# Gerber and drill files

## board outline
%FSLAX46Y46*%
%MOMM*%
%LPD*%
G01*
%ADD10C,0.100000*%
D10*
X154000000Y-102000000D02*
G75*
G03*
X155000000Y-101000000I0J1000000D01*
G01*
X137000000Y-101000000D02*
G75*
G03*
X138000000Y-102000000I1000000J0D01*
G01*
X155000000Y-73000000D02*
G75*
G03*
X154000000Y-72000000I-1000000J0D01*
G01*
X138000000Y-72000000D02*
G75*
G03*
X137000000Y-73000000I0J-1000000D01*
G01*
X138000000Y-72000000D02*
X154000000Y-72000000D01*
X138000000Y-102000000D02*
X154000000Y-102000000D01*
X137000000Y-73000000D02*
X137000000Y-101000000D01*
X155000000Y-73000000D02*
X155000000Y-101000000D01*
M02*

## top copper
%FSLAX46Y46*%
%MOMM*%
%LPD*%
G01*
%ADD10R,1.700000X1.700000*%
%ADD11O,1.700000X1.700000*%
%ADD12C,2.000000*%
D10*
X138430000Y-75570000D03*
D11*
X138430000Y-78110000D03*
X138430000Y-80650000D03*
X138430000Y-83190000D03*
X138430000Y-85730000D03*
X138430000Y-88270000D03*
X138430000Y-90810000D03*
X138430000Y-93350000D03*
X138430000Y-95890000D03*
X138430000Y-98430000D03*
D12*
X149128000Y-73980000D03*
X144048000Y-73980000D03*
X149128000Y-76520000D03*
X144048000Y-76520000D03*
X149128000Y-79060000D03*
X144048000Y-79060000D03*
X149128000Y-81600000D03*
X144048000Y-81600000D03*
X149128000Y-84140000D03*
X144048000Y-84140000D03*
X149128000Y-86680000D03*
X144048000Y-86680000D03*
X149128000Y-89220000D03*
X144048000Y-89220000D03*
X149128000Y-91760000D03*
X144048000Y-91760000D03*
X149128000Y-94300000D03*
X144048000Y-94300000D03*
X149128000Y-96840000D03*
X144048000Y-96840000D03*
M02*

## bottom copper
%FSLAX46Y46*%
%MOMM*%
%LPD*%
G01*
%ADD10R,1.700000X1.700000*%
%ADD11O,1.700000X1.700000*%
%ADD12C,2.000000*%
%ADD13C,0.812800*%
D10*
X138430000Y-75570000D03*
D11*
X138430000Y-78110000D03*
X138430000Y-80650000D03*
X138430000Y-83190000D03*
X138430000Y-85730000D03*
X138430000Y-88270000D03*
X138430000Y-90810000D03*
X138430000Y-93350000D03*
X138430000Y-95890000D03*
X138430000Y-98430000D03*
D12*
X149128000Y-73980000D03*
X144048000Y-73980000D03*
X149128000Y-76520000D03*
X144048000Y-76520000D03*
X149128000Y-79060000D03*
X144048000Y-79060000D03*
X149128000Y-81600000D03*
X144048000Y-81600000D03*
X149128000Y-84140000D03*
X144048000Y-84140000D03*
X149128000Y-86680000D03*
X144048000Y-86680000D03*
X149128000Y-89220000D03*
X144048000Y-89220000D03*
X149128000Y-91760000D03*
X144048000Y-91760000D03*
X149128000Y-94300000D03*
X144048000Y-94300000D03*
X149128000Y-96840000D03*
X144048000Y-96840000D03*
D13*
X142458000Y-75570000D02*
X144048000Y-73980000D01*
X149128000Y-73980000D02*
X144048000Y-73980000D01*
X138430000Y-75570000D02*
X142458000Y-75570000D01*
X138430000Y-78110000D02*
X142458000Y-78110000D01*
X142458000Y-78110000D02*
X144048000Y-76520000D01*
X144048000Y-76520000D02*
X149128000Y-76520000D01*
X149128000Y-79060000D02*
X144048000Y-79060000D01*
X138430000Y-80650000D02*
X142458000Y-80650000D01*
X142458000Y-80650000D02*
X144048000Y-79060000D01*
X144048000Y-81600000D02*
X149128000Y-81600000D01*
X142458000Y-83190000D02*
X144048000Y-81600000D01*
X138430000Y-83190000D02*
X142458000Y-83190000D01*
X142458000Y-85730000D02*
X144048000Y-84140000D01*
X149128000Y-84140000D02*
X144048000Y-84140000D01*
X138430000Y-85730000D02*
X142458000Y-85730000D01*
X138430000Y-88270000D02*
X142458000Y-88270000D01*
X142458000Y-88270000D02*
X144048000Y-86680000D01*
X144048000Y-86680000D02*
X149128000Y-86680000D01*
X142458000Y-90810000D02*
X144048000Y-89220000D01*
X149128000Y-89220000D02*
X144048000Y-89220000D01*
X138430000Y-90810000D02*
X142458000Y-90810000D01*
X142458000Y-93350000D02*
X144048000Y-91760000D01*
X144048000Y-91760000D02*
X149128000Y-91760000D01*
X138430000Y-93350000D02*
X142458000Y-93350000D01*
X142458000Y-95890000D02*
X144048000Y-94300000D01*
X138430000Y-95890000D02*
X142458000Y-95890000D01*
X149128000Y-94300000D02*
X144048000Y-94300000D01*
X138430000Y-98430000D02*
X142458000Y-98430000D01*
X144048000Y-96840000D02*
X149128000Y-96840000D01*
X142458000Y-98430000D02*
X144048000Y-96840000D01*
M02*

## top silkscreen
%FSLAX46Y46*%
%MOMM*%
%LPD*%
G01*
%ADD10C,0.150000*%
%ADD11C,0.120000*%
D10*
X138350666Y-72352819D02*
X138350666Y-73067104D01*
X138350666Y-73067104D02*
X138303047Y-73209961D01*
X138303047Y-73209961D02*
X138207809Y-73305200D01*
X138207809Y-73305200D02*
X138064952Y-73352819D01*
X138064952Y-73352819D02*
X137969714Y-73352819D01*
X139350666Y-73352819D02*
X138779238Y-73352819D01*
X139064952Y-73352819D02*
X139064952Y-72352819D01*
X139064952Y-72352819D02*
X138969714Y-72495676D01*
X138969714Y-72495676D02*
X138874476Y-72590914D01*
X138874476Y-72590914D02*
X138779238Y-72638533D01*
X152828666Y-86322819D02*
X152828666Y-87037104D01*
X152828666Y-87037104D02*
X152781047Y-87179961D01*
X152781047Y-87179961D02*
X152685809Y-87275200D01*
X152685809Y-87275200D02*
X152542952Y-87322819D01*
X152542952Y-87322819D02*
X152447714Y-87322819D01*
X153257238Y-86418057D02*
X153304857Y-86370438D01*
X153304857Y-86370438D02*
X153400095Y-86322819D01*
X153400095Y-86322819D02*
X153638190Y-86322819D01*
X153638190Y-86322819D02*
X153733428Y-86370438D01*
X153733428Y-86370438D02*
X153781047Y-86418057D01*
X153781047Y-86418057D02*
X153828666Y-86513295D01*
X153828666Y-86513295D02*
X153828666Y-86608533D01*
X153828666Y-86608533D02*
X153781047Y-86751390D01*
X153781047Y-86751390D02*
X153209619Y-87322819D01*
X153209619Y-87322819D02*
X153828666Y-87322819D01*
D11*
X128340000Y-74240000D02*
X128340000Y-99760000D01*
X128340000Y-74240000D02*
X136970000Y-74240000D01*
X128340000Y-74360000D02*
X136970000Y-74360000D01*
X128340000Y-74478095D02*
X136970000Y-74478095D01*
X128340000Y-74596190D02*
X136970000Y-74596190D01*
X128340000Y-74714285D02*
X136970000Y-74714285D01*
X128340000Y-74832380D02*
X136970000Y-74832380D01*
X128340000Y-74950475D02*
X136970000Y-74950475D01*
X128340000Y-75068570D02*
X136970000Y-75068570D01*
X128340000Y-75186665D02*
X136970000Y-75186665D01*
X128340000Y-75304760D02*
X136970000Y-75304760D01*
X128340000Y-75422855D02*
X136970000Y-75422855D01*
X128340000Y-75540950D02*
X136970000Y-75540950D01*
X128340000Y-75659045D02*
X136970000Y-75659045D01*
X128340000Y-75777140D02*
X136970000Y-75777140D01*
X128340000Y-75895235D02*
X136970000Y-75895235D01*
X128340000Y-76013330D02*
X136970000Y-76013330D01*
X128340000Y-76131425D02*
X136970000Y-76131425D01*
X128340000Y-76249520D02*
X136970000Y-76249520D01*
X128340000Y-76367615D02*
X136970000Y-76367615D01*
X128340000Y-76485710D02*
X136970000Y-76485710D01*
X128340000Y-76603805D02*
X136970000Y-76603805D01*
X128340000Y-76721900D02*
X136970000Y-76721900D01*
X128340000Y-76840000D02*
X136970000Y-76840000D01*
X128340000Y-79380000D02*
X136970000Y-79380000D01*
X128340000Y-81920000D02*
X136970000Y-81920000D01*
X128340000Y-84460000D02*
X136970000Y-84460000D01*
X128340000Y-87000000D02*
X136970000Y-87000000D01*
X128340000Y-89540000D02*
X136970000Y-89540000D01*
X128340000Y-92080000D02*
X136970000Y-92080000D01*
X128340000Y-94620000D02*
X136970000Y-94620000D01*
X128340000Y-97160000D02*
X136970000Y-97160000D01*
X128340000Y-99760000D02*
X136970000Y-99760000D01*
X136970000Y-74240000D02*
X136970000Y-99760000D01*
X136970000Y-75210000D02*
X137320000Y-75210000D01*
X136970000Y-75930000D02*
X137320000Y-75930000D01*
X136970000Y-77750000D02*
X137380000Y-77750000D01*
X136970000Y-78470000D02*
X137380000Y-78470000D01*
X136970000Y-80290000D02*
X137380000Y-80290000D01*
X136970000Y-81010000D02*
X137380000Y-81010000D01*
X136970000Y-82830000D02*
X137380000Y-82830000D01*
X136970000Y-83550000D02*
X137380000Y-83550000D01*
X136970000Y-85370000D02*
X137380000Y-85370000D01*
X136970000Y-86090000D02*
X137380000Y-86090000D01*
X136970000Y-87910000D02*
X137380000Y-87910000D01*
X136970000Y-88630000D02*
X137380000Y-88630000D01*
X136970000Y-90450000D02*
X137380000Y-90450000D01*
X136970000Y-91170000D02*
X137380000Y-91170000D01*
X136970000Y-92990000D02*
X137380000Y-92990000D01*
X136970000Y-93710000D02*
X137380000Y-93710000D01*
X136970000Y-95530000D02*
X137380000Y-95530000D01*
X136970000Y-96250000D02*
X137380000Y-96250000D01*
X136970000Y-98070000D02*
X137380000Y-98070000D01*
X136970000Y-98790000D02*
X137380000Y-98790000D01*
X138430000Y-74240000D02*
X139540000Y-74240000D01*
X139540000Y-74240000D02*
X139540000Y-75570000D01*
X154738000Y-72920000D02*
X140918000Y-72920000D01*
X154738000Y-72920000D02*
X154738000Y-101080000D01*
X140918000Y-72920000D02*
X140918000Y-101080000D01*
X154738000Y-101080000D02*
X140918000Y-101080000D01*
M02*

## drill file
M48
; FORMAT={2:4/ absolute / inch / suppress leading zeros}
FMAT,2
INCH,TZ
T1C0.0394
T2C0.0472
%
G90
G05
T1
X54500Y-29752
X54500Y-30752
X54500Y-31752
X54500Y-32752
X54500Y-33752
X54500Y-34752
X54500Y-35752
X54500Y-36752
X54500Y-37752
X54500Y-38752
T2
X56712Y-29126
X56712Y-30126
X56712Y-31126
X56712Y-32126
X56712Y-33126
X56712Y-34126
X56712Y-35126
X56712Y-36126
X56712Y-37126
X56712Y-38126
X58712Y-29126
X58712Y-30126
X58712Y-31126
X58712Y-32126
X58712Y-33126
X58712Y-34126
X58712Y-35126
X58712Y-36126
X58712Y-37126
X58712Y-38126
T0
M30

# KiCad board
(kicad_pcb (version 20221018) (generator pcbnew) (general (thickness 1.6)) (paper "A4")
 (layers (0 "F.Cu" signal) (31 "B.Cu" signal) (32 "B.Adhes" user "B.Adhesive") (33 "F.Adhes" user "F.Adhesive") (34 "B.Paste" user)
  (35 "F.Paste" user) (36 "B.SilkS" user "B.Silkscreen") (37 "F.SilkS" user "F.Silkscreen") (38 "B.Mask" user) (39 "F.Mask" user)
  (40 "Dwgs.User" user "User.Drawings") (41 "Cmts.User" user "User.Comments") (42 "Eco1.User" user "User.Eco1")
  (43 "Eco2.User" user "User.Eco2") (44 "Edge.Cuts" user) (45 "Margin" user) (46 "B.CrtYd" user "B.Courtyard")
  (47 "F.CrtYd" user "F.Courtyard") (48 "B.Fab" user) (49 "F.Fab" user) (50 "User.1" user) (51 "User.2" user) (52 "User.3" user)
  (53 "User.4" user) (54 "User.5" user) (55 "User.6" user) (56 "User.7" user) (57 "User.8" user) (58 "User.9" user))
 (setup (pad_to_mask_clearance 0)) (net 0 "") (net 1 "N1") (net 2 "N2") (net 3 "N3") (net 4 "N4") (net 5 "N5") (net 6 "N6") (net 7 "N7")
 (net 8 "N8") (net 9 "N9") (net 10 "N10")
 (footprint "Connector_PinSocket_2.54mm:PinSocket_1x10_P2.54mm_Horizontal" (layer "F.Cu") (at 138.43 75.57)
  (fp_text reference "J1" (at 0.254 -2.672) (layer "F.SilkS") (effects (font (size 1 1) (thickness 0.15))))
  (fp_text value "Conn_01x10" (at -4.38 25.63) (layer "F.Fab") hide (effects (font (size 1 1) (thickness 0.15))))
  (fp_line (start -10.09 -1.33) (end -10.09 24.19) (stroke (width 0.12) (type solid)) (layer "F.SilkS"))
  (fp_line (start -10.09 -1.33) (end -1.46 -1.33) (stroke (width 0.12) (type solid)) (layer "F.SilkS"))
  (fp_line (start -10.09 -1.21) (end -1.46 -1.21) (stroke (width 0.12) (type solid)) (layer "F.SilkS"))
  (fp_line (start -10.09 -1.091905) (end -1.46 -1.091905) (stroke (width 0.12) (type solid)) (layer "F.SilkS"))
  (fp_line (start -10.09 -0.97381) (end -1.46 -0.97381) (stroke (width 0.12) (type solid)) (layer "F.SilkS"))
  (fp_line (start -10.09 -0.855715) (end -1.46 -0.855715) (stroke (width 0.12) (type solid)) (layer "F.SilkS"))
  (fp_line (start -10.09 -0.73762) (end -1.46 -0.73762) (stroke (width 0.12) (type solid)) (layer "F.SilkS"))
  (fp_line (start -10.09 -0.619525) (end -1.46 -0.619525) (stroke (width 0.12) (type solid)) (layer "F.SilkS"))
  (fp_line (start -10.09 -0.50143) (end -1.46 -0.50143) (stroke (width 0.12) (type solid)) (layer "F.SilkS"))
  (fp_line (start -10.09 -0.383335) (end -1.46 -0.383335) (stroke (width 0.12) (type solid)) (layer "F.SilkS"))
  (fp_line (start -10.09 -0.26524) (end -1.46 -0.26524) (stroke (width 0.12) (type solid)) (layer "F.SilkS"))
  (fp_line (start -10.09 -0.147145) (end -1.46 -0.147145) (stroke (width 0.12) (type solid)) (layer "F.SilkS"))
  (fp_line (start -10.09 -0.02905) (end -1.46 -0.02905) (stroke (width 0.12) (type solid)) (layer "F.SilkS"))
  (fp_line (start -10.09 0.089045) (end -1.46 0.089045) (stroke (width 0.12) (type solid)) (layer "F.SilkS"))
  (fp_line (start -10.09 0.20714) (end -1.46 0.20714) (stroke (width 0.12) (type solid)) (layer "F.SilkS"))
  (fp_line (start -10.09 0.325235) (end -1.46 0.325235) (stroke (width 0.12) (type solid)) (layer "F.SilkS"))
  (fp_line (start -10.09 0.44333) (end -1.46 0.44333) (stroke (width 0.12) (type solid)) (layer "F.SilkS"))
  (fp_line (start -10.09 0.561425) (end -1.46 0.561425) (stroke (width 0.12) (type solid)) (layer "F.SilkS"))
  (fp_line (start -10.09 0.67952) (end -1.46 0.67952) (stroke (width 0.12) (type solid)) (layer "F.SilkS"))
  (fp_line (start -10.09 0.797615) (end -1.46 0.797615) (stroke (width 0.12) (type solid)) (layer "F.SilkS"))
  (fp_line (start -10.09 0.91571) (end -1.46 0.91571) (stroke (width 0.12) (type solid)) (layer "F.SilkS"))
  (fp_line (start -10.09 1.033805) (end -1.46 1.033805) (stroke (width 0.12) (type solid)) (layer "F.SilkS"))
  (fp_line (start -10.09 1.1519) (end -1.46 1.1519) (stroke (width 0.12) (type solid)) (layer "F.SilkS"))
  (fp_line (start -10.09 1.27) (end -1.46 1.27) (stroke (width 0.12) (type solid)) (layer "F.SilkS"))
  (fp_line (start -10.09 3.81) (end -1.46 3.81) (stroke (width 0.12) (type solid)) (layer "F.SilkS"))
  (fp_line (start -10.09 6.35) (end -1.46 6.35) (stroke (width 0.12) (type solid)) (layer "F.SilkS"))
  (fp_line (start -10.09 8.89) (end -1.46 8.89) (stroke (width 0.12) (type solid)) (layer "F.SilkS"))
  (fp_line (start -10.09 11.43) (end -1.46 11.43) (stroke (width 0.12) (type solid)) (layer "F.SilkS"))
  (fp_line (start -10.09 13.97) (end -1.46 13.97) (stroke (width 0.12) (type solid)) (layer "F.SilkS"))
  (fp_line (start -10.09 16.51) (end -1.46 16.51) (stroke (width 0.12) (type solid)) (layer "F.SilkS"))
  (fp_line (start -10.09 19.05) (end -1.46 19.05) (stroke (width 0.12) (type solid)) (layer "F.SilkS"))
  (fp_line (start -10.09 21.59) (end -1.46 21.59) (stroke (width 0.12) (type solid)) (layer "F.SilkS"))
  (fp_line (start -10.09 24.19) (end -1.46 24.19) (stroke (width 0.12) (type solid)) (layer "F.SilkS"))
  (fp_line (start -1.46 -1.33) (end -1.46 24.19) (stroke (width 0.12) (type solid)) (layer "F.SilkS"))
  (fp_line (start -1.46 -0.36) (end -1.11 -0.36) (stroke (width 0.12) (type solid)) (layer "F.SilkS"))
  (fp_line (start -1.46 0.36) (end -1.11 0.36) (stroke (width 0.12) (type solid)) (layer "F.SilkS"))
  (fp_line (start -1.46 2.18) (end -1.05 2.18) (stroke (width 0.12) (type solid)) (layer "F.SilkS"))
  (fp_line (start -1.46 2.9) (end -1.05 2.9) (stroke (width 0.12) (type solid)) (layer "F.SilkS"))
  (fp_line (start -1.46 4.72) (end -1.05 4.72) (stroke (width 0.12) (type solid)) (layer "F.SilkS"))
  (fp_line (start -1.46 5.44) (end -1.05 5.44) (stroke (width 0.12) (type solid)) (layer "F.SilkS"))
  (fp_line (start -1.46 7.26) (end -1.05 7.26) (stroke (width 0.12) (type solid)) (layer "F.SilkS"))
  (fp_line (start -1.46 7.98) (end -1.05 7.98) (stroke (width 0.12) (type solid)) (layer "F.SilkS"))
  (fp_line (start -1.46 9.8) (end -1.05 9.8) (stroke (width 0.12) (type solid)) (layer "F.SilkS"))
  (fp_line (start -1.46 10.52) (end -1.05 10.52) (stroke (width 0.12) (type solid)) (layer "F.SilkS"))
  (fp_line (start -1.46 12.34) (end -1.05 12.34) (stroke (width 0.12) (type solid)) (layer "F.SilkS"))
  (fp_line (start -1.46 13.06) (end -1.05 13.06) (stroke (width 0.12) (type solid)) (layer "F.SilkS"))
  (fp_line (start -1.46 14.88) (end -1.05 14.88) (stroke (width 0.12) (type solid)) (layer "F.SilkS"))
  (fp_line (start -1.46 15.6) (end -1.05 15.6) (stroke (width 0.12) (type solid)) (layer "F.SilkS"))
  (fp_line (start -1.46 17.42) (end -1.05 17.42) (stroke (width 0.12) (type solid)) (layer "F.SilkS"))
  (fp_line (start -1.46 18.14) (end -1.05 18.14) (stroke (width 0.12) (type solid)) (layer "F.SilkS"))
  (fp_line (start -1.46 19.96) (end -1.05 19.96) (stroke (width 0.12) (type solid)) (layer "F.SilkS"))
  (fp_line (start -1.46 20.68) (end -1.05 20.68) (stroke (width 0.12) (type solid)) (layer "F.SilkS"))
  (fp_line (start -1.46 22.5) (end -1.05 22.5) (stroke (width 0.12) (type solid)) (layer "F.SilkS"))
  (fp_line (start -1.46 23.22) (end -1.05 23.22) (stroke (width 0.12) (type solid)) (layer "F.SilkS"))
  (fp_line (start 0 -1.33) (end 1.11 -1.33) (stroke (width 0.12) (type solid)) (layer "F.SilkS"))
  (fp_line (start 1.11 -1.33) (end 1.11 0) (stroke (width 0.12) (type solid)) (layer "F.SilkS"))
  (pad "1" thru_hole rect (at 0 0) (size 1.7 1.7) (drill 1) (layers "*.Cu" "*.Mask") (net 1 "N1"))
  (pad "2" thru_hole oval (at 0 2.54) (size 1.7 1.7) (drill 1) (layers "*.Cu" "*.Mask") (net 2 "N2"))
  (pad "3" thru_hole oval (at 0 5.08) (size 1.7 1.7) (drill 1) (layers "*.Cu" "*.Mask") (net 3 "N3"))
  (pad "4" thru_hole oval (at 0 7.62) (size 1.7 1.7) (drill 1) (layers "*.Cu" "*.Mask") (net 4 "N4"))
  (pad "5" thru_hole oval (at 0 10.16) (size 1.7 1.7) (drill 1) (layers "*.Cu" "*.Mask") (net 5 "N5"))
  (pad "6" thru_hole oval (at 0 12.7) (size 1.7 1.7) (drill 1) (layers "*.Cu" "*.Mask") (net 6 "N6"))
  (pad "7" thru_hole oval (at 0 15.24) (size 1.7 1.7) (drill 1) (layers "*.Cu" "*.Mask") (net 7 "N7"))
  (pad "8" thru_hole oval (at 0 17.78) (size 1.7 1.7) (drill 1) (layers "*.Cu" "*.Mask") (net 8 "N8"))
  (pad "9" thru_hole oval (at 0 20.32) (size 1.7 1.7) (drill 1) (layers "*.Cu" "*.Mask") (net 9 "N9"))
  (pad "10" thru_hole oval (at 0 22.86) (size 1.7 1.7) (drill 1) (layers "*.Cu" "*.Mask") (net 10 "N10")))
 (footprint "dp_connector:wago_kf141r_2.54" (layer "F.Cu") (at 147.828 87 -90)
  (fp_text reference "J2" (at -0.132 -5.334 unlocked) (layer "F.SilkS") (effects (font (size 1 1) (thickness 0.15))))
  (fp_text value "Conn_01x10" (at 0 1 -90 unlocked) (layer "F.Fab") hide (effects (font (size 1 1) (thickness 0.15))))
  (fp_line (start -14.08 -6.91) (end -14.08 6.91) (stroke (width 0.12) (type default)) (layer "F.SilkS"))
  (fp_line (start -14.08 -6.91) (end 14.08 -6.91) (stroke (width 0.12) (type default)) (layer "F.SilkS"))
  (fp_line (start -14.08 6.91) (end 14.08 6.91) (stroke (width 0.12) (type default)) (layer "F.SilkS"))
  (fp_line (start 14.08 -6.91) (end 14.08 6.91) (stroke (width 0.12) (type default)) (layer "F.SilkS"))
  (pad "1" thru_hole circle (at -13.02 -1.3 270) (size 2 2) (drill 1.2) (layers "*.Cu" "*.Mask") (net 1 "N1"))
  (pad "1" thru_hole circle (at -13.02 3.78 270) (size 2 2) (drill 1.2) (layers "*.Cu" "*.Mask") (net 1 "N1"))
  (pad "2" thru_hole circle (at -10.48 -1.3 270) (size 2 2) (drill 1.2) (layers "*.Cu" "*.Mask") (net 2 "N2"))
  (pad "2" thru_hole circle (at -10.48 3.78 270) (size 2 2) (drill 1.2) (layers "*.Cu" "*.Mask") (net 2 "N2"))
  (pad "3" thru_hole circle (at -7.94 -1.3 270) (size 2 2) (drill 1.2) (layers "*.Cu" "*.Mask") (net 3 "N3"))
  (pad "3" thru_hole circle (at -7.94 3.78 270) (size 2 2) (drill 1.2) (layers "*.Cu" "*.Mask") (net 3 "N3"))
  (pad "4" thru_hole circle (at -5.4 -1.3 270) (size 2 2) (drill 1.2) (layers "*.Cu" "*.Mask") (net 4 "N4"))
  (pad "4" thru_hole circle (at -5.4 3.78 270) (size 2 2) (drill 1.2) (layers "*.Cu" "*.Mask") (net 4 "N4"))
  (pad "5" thru_hole circle (at -2.86 -1.3 270) (size 2 2) (drill 1.2) (layers "*.Cu" "*.Mask") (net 5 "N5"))
  (pad "5" thru_hole circle (at -2.86 3.78 270) (size 2 2) (drill 1.2) (layers "*.Cu" "*.Mask") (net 5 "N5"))
  (pad "6" thru_hole circle (at -0.32 -1.3 270) (size 2 2) (drill 1.2) (layers "*.Cu" "*.Mask") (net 6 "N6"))
  (pad "6" thru_hole circle (at -0.32 3.78 270) (size 2 2) (drill 1.2) (layers "*.Cu" "*.Mask") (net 6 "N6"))
  (pad "7" thru_hole circle (at 2.22 -1.3 270) (size 2 2) (drill 1.2) (layers "*.Cu" "*.Mask") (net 7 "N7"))
  (pad "7" thru_hole circle (at 2.22 3.78 270) (size 2 2) (drill 1.2) (layers "*.Cu" "*.Mask") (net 7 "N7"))
  (pad "8" thru_hole circle (at 4.76 -1.3 270) (size 2 2) (drill 1.2) (layers "*.Cu" "*.Mask") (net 8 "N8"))
  (pad "8" thru_hole circle (at 4.76 3.78 270) (size 2 2) (drill 1.2) (layers "*.Cu" "*.Mask") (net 8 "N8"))
  (pad "9" thru_hole circle (at 7.3 -1.3 270) (size 2 2) (drill 1.2) (layers "*.Cu" "*.Mask") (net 9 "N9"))
  (pad "9" thru_hole circle (at 7.3 3.78 270) (size 2 2) (drill 1.2) (layers "*.Cu" "*.Mask") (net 9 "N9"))
  (pad "10" thru_hole circle (at 9.84 -1.3 270) (size 2 2) (drill 1.2) (layers "*.Cu" "*.Mask") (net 10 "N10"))
  (pad "10" thru_hole circle (at 9.84 3.78 270) (size 2 2) (drill 1.2) (layers "*.Cu" "*.Mask") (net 10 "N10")))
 (gr_line (start 138 72) (end 154 72) (stroke (width 0.1) (type default)) (layer "Edge.Cuts"))
 (gr_line (start 138 102) (end 154 102) (stroke (width 0.1) (type default)) (layer "Edge.Cuts"))
 (gr_line (start 137 73) (end 137 101) (stroke (width 0.1) (type default)) (layer "Edge.Cuts"))
 (gr_arc (start 155 101) (mid 154.707107 101.707107) (end 154 102) (stroke (width 0.1) (type default)) (layer "Edge.Cuts"))
 (gr_arc (start 154 72) (mid 154.707107 72.292893) (end 155 73) (stroke (width 0.1) (type default)) (layer "Edge.Cuts"))
 (gr_line (start 155 73) (end 155 101) (stroke (width 0.1) (type default)) (layer "Edge.Cuts"))
 (gr_arc (start 138 102) (mid 137.292893 101.707107) (end 137 101) (stroke (width 0.1) (type default)) (layer "Edge.Cuts"))
 (gr_arc (start 137 73) (mid 137.292893 72.292893) (end 138 72) (stroke (width 0.1) (type default)) (layer "Edge.Cuts"))
 (segment (start 142.458 75.57) (end 144.048 73.98) (width 0.8128) (layer "B.Cu") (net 1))
 (segment (start 149.128 73.98) (end 144.048 73.98) (width 0.8128) (layer "B.Cu") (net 1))
 (segment (start 138.43 75.57) (end 142.458 75.57) (width 0.8128) (layer "B.Cu") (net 1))
 (segment (start 138.43 78.11) (end 142.458 78.11) (width 0.8128) (layer "B.Cu") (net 2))
 (segment (start 142.458 78.11) (end 144.048 76.52) (width 0.8128) (layer "B.Cu") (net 2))
 (segment (start 144.048 76.52) (end 149.128 76.52) (width 0.8128) (layer "B.Cu") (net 2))
 (segment (start 149.128 79.06) (end 144.048 79.06) (width 0.8128) (layer "B.Cu") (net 3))
 (segment (start 138.43 80.65) (end 142.458 80.65) (width 0.8128) (layer "B.Cu") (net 3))
 (segment (start 142.458 80.65) (end 144.048 79.06) (width 0.8128) (layer "B.Cu") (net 3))
 (segment (start 144.048 81.6) (end 149.128 81.6) (width 0.8128) (layer "B.Cu") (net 4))
 (segment (start 142.458 83.19) (end 144.048 81.6) (width 0.8128) (layer "B.Cu") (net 4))
 (segment (start 138.43 83.19) (end 142.458 83.19) (width 0.8128) (layer "B.Cu") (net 4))
 (segment (start 142.458 85.73) (end 144.048 84.14) (width 0.8128) (layer "B.Cu") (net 5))
 (segment (start 149.128 84.14) (end 144.048 84.14) (width 0.8128) (layer "B.Cu") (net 5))
 (segment (start 138.43 85.73) (end 142.458 85.73) (width 0.8128) (layer "B.Cu") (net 5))
 (segment (start 138.43 88.27) (end 142.458 88.27) (width 0.8128) (layer "B.Cu") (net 6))
 (segment (start 142.458 88.27) (end 144.048 86.68) (width 0.8128) (layer "B.Cu") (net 6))
 (segment (start 144.048 86.68) (end 149.128 86.68) (width 0.8128) (layer "B.Cu") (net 6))
 (segment (start 142.458 90.81) (end 144.048 89.22) (width 0.8128) (layer "B.Cu") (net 7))
 (segment (start 149.128 89.22) (end 144.048 89.22) (width 0.8128) (layer "B.Cu") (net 7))
 (segment (start 138.43 90.81) (end 142.458 90.81) (width 0.8128) (layer "B.Cu") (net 7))
 (segment (start 142.458 93.35) (end 144.048 91.76) (width 0.8128) (layer "B.Cu") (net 8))
 (segment (start 144.048 91.76) (end 149.128 91.76) (width 0.8128) (layer "B.Cu") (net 8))
 (segment (start 138.43 93.35) (end 142.458 93.35) (width 0.8128) (layer "B.Cu") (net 8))
 (segment (start 142.458 95.89) (end 144.048 94.3) (width 0.8128) (layer "B.Cu") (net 9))
 (segment (start 138.43 95.89) (end 142.458 95.89) (width 0.8128) (layer "B.Cu") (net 9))
 (segment (start 149.128 94.3) (end 144.048 94.3) (width 0.8128) (layer "B.Cu") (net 9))
 (segment (start 138.43 98.43) (end 142.458 98.43) (width 0.8128) (layer "B.Cu") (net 10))
 (segment (start 144.048 96.84) (end 149.128 96.84) (width 0.8128) (layer "B.Cu") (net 10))
 (segment (start 142.458 98.43) (end 144.048 96.84) (width 0.8128) (layer "B.Cu") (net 10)))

